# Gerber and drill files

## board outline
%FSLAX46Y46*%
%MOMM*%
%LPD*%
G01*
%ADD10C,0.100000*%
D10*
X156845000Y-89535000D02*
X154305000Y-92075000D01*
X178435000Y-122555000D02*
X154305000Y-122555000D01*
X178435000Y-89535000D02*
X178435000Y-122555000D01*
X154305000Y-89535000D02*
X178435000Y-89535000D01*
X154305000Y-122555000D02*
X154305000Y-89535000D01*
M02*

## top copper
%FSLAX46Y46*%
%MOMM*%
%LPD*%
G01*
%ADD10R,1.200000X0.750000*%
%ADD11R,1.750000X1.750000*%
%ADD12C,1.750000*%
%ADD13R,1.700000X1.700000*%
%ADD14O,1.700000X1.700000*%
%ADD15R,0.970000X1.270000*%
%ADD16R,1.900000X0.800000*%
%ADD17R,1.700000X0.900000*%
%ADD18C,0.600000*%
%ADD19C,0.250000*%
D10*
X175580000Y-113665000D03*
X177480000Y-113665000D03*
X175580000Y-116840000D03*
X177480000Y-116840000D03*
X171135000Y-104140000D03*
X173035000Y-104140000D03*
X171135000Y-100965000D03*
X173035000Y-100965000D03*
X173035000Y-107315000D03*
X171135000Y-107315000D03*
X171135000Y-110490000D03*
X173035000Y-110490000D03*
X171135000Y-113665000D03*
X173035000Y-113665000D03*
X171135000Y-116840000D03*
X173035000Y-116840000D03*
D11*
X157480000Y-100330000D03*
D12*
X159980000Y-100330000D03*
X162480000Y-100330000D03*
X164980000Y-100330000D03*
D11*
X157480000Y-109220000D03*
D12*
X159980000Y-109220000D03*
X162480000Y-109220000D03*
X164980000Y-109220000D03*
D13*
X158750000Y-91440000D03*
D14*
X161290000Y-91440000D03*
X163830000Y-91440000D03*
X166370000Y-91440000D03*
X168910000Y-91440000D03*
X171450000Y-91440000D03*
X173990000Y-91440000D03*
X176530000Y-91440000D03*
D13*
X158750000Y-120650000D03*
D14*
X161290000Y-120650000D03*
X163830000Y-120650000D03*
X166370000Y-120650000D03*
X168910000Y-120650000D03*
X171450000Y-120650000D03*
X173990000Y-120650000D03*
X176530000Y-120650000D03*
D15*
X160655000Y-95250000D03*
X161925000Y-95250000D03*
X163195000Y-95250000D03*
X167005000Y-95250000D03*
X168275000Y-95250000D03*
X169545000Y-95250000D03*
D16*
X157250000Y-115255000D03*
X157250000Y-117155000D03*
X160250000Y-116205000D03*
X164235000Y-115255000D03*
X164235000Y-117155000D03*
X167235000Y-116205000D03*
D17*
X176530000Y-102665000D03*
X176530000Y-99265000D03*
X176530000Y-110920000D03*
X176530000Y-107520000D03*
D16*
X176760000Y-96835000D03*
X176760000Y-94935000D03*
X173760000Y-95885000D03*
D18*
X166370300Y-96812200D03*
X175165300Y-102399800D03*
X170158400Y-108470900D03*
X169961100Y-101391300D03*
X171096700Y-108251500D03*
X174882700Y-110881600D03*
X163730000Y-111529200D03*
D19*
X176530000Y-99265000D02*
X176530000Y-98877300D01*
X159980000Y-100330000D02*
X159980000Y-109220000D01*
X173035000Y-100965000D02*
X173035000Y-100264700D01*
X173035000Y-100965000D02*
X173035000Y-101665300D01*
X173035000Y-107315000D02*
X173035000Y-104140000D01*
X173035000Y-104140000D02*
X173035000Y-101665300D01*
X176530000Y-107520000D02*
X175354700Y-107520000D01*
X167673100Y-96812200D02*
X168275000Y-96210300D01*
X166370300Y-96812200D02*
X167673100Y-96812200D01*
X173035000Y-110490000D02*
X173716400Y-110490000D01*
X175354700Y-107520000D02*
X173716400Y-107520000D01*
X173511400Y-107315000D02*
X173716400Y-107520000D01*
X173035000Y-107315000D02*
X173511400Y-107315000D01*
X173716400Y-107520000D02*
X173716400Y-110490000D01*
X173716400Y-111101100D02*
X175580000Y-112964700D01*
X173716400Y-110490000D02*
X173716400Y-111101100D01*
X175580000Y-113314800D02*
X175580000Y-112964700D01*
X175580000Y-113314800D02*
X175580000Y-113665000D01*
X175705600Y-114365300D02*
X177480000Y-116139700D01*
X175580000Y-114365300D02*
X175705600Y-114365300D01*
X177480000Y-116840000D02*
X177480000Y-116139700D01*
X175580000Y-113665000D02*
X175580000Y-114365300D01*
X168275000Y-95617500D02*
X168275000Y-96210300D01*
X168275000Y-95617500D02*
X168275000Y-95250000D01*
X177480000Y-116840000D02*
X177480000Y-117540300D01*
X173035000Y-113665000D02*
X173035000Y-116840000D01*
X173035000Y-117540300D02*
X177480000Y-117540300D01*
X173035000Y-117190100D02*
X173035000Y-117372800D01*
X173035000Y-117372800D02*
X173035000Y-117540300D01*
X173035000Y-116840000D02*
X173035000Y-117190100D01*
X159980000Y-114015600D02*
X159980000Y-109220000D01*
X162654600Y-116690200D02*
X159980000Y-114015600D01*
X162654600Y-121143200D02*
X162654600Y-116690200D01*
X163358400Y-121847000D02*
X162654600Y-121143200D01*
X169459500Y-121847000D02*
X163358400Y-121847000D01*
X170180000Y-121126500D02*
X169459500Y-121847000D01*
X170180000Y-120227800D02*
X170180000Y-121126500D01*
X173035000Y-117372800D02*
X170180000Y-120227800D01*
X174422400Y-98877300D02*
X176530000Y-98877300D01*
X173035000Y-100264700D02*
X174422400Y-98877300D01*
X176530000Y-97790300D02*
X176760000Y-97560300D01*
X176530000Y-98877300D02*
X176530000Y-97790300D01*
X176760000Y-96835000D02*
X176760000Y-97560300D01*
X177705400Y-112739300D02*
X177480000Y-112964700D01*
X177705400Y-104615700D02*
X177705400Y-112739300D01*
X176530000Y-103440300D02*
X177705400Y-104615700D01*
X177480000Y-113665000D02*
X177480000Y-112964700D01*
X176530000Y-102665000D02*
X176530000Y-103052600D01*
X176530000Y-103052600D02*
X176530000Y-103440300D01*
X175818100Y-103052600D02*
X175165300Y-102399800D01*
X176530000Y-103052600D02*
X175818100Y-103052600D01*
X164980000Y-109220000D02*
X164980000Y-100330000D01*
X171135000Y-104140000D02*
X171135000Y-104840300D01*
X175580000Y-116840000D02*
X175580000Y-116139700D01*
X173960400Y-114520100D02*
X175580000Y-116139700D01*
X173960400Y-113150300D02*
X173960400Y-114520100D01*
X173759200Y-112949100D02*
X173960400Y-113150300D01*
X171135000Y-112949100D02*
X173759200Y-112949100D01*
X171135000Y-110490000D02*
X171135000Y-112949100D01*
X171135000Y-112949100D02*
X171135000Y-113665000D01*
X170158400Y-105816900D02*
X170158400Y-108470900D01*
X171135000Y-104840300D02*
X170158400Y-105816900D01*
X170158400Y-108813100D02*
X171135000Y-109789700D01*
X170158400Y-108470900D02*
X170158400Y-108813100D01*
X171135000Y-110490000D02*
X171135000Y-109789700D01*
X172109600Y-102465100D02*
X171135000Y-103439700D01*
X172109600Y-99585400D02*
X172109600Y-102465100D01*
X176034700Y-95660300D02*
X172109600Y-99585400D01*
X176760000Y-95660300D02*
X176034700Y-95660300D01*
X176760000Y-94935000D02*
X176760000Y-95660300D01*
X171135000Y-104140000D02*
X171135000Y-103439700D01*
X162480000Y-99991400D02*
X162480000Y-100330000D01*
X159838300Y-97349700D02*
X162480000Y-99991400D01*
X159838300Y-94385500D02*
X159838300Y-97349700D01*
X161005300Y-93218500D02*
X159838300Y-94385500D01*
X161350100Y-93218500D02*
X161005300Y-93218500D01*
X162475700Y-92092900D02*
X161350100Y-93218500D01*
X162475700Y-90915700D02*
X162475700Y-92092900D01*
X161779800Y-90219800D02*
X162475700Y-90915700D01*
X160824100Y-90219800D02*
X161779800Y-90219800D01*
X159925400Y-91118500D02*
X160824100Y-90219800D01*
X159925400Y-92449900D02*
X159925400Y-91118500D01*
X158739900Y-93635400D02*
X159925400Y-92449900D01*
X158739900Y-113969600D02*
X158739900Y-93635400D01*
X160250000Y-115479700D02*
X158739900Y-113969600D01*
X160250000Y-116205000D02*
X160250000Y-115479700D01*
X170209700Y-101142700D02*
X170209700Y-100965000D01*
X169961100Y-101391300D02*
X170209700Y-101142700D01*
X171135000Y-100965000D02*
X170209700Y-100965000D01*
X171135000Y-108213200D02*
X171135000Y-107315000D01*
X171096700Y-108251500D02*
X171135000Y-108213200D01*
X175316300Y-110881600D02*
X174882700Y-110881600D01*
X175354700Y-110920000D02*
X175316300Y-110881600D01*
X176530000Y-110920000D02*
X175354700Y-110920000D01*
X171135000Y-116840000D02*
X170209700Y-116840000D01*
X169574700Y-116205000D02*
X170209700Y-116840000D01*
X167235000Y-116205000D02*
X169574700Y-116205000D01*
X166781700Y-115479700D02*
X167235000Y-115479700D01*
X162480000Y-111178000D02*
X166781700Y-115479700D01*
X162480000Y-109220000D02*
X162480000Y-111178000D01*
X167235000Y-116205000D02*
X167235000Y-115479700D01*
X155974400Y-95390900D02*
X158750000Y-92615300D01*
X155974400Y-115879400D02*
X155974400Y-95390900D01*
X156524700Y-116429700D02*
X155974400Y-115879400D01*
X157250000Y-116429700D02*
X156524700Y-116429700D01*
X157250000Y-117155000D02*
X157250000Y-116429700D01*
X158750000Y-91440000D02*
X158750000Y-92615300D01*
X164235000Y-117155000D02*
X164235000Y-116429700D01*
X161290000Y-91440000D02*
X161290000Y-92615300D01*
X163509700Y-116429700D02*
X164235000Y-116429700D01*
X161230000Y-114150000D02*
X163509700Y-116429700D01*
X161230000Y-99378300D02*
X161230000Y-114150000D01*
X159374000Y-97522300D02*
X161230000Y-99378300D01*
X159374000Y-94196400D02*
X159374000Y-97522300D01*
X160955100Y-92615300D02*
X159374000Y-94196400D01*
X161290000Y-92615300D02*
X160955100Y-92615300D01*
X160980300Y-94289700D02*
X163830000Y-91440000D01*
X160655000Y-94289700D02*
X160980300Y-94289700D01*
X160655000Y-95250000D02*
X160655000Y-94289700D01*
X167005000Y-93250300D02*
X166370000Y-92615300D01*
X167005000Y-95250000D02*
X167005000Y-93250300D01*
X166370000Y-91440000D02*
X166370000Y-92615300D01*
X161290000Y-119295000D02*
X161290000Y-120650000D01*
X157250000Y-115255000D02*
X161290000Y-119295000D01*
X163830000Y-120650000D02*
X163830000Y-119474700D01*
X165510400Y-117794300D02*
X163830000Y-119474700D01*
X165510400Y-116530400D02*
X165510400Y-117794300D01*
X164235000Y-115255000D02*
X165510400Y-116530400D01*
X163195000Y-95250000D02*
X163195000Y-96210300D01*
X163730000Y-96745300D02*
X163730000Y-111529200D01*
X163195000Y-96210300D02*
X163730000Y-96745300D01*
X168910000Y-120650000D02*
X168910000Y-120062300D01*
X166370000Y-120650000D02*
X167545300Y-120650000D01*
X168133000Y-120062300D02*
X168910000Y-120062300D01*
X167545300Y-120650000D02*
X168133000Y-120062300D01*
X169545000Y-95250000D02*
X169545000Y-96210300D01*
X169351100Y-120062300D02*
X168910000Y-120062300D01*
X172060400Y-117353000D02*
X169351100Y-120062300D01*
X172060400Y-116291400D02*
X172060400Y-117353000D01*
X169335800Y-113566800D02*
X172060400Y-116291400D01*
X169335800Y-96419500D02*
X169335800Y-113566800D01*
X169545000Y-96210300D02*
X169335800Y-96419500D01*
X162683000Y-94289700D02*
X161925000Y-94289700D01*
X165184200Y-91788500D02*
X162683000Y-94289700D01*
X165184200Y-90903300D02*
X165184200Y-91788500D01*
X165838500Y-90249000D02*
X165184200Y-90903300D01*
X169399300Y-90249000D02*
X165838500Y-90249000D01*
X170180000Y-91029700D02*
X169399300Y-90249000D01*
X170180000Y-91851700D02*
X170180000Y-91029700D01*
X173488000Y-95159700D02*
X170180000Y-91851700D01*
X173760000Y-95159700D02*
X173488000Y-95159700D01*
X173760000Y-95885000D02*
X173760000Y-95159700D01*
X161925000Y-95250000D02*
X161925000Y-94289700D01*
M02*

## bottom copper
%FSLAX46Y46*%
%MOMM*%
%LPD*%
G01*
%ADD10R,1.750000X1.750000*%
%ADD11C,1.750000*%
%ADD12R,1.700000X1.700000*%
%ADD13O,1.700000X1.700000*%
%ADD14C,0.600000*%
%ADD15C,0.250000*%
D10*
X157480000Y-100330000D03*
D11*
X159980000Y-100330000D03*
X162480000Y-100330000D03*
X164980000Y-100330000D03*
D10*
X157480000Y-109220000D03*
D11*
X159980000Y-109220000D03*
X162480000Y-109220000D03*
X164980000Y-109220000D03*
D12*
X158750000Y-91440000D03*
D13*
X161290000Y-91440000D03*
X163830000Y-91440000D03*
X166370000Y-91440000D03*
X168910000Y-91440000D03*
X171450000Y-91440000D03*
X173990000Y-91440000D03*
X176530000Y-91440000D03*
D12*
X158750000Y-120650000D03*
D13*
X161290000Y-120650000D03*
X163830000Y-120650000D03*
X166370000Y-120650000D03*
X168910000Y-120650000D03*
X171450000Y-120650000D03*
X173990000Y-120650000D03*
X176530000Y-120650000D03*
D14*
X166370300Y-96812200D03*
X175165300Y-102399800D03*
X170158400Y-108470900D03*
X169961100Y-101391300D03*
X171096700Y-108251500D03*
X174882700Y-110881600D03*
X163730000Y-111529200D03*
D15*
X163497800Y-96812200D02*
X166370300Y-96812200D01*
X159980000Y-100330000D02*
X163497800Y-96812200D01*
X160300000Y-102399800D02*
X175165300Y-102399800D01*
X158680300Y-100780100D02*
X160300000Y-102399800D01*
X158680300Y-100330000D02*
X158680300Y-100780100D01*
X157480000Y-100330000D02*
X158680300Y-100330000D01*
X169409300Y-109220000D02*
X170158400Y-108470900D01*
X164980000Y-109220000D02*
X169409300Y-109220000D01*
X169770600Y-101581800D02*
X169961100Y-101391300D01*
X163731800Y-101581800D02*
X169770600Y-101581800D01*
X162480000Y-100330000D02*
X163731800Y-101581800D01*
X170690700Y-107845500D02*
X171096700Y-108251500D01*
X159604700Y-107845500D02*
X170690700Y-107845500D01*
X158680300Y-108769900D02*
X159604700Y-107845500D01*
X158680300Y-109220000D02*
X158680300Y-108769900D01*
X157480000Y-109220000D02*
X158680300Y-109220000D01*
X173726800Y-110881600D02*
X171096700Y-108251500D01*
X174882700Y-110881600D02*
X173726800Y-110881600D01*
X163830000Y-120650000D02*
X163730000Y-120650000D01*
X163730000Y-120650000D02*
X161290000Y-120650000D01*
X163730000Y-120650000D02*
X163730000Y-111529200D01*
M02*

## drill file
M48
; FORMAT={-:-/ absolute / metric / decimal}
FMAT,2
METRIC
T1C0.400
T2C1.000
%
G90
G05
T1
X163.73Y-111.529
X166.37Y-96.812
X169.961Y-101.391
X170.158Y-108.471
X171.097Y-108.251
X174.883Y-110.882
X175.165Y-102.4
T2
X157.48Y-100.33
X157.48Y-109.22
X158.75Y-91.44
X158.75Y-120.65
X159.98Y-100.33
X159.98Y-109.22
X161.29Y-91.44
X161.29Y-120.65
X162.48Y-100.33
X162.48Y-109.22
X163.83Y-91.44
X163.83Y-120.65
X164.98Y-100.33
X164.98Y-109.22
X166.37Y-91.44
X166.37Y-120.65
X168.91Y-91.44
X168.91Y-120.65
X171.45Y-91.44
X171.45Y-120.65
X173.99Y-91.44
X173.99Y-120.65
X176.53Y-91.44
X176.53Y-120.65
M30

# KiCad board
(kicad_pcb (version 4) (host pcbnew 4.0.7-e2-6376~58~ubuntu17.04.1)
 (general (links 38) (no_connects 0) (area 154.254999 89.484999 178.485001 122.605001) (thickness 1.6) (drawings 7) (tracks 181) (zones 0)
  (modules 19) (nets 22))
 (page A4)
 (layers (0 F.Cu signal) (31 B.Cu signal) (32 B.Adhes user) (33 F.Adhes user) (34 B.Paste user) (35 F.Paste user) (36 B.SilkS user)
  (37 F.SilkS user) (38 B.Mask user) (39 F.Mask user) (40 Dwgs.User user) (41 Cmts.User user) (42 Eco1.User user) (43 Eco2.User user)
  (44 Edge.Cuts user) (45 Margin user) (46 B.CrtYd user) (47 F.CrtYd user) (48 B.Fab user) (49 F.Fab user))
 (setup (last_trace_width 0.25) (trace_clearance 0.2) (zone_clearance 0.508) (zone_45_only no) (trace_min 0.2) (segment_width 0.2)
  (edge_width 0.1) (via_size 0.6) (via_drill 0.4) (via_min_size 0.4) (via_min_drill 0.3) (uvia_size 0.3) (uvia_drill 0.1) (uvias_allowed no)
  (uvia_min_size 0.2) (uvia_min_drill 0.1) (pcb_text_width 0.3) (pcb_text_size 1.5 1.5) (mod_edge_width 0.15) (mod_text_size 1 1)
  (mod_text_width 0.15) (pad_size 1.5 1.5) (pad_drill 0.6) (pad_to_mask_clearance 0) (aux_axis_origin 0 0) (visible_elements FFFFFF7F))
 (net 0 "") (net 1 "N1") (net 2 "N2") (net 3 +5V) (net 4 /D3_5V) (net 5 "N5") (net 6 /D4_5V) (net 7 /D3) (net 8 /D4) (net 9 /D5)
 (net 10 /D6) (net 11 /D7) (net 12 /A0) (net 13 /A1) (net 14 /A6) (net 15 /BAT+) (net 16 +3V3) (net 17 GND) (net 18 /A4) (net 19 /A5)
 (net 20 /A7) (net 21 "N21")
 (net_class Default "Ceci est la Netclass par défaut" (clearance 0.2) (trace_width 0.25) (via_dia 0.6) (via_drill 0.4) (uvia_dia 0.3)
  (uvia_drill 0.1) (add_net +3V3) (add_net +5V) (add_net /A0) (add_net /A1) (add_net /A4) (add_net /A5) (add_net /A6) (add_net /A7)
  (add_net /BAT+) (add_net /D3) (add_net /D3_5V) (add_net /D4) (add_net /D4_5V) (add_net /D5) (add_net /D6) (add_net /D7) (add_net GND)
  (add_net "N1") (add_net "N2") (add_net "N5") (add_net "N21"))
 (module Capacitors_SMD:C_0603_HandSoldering (layer F.Cu) (at 176.53 113.665)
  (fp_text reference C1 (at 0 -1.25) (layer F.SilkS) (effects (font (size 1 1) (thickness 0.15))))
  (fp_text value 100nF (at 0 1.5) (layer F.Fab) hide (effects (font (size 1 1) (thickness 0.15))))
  (pad 1 smd rect (at -0.95 0) (size 1.2 0.75) (layers F.Cu F.Paste F.Mask) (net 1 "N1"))
  (pad 2 smd rect (at 0.95 0) (size 1.2 0.75) (layers F.Cu F.Paste F.Mask) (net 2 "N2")))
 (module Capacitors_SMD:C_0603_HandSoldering (layer F.Cu) (at 176.53 116.84)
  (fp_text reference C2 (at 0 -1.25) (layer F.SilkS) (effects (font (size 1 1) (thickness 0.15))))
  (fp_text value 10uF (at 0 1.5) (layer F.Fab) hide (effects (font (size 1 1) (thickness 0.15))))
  (pad 1 smd rect (at -0.95 0) (size 1.2 0.75) (layers F.Cu F.Paste F.Mask) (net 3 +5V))
  (pad 2 smd rect (at 0.95 0) (size 1.2 0.75) (layers F.Cu F.Paste F.Mask) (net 1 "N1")))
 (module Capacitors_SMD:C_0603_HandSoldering (layer F.Cu) (at 172.085 104.14)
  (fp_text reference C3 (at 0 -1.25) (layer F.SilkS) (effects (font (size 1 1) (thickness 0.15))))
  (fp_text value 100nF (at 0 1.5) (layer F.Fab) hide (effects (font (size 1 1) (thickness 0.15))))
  (pad 1 smd rect (at -0.95 0) (size 1.2 0.75) (layers F.Cu F.Paste F.Mask) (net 3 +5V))
  (pad 2 smd rect (at 0.95 0) (size 1.2 0.75) (layers F.Cu F.Paste F.Mask) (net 1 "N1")))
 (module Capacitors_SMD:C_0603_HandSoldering (layer F.Cu) (at 172.085 100.965)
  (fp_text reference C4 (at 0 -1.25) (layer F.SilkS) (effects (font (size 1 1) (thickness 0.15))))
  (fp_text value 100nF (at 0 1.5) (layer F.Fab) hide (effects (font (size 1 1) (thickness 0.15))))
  (pad 1 smd rect (at -0.95 0) (size 1.2 0.75) (layers F.Cu F.Paste F.Mask) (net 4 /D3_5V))
  (pad 2 smd rect (at 0.95 0) (size 1.2 0.75) (layers F.Cu F.Paste F.Mask) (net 1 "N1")))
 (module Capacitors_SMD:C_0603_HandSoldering (layer F.Cu) (at 172.085 107.315 180)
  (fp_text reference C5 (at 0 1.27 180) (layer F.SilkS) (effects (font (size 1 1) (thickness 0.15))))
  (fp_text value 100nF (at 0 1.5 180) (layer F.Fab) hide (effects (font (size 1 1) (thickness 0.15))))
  (pad 1 smd rect (at -0.95 0 180) (size 1.2 0.75) (layers F.Cu F.Paste F.Mask) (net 1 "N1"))
  (pad 2 smd rect (at 0.95 0 180) (size 1.2 0.75) (layers F.Cu F.Paste F.Mask) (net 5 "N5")))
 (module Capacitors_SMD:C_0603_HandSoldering (layer F.Cu) (at 172.085 110.49)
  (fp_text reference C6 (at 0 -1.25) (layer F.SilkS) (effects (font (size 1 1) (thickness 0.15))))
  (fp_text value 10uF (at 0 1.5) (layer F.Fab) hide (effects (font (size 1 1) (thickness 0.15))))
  (pad 1 smd rect (at -0.95 0) (size 1.2 0.75) (layers F.Cu F.Paste F.Mask) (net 3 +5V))
  (pad 2 smd rect (at 0.95 0) (size 1.2 0.75) (layers F.Cu F.Paste F.Mask) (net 1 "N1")))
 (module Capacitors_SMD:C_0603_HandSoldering (layer F.Cu) (at 172.085 113.665)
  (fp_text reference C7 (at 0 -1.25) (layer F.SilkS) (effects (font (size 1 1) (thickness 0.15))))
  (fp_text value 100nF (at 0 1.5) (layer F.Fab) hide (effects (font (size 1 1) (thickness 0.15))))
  (pad 1 smd rect (at -0.95 0) (size 1.2 0.75) (layers F.Cu F.Paste F.Mask) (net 3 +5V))
  (pad 2 smd rect (at 0.95 0) (size 1.2 0.75) (layers F.Cu F.Paste F.Mask) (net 1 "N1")))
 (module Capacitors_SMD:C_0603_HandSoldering (layer F.Cu) (at 172.085 116.84)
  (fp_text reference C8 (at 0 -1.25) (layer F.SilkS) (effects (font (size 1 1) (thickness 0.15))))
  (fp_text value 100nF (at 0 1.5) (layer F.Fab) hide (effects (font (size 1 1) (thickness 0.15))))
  (pad 1 smd rect (at -0.95 0) (size 1.2 0.75) (layers F.Cu F.Paste F.Mask) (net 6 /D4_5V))
  (pad 2 smd rect (at 0.95 0) (size 1.2 0.75) (layers F.Cu F.Paste F.Mask) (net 1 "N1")))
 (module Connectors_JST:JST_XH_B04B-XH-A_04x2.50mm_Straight (layer F.Cu) (at 157.48 100.33)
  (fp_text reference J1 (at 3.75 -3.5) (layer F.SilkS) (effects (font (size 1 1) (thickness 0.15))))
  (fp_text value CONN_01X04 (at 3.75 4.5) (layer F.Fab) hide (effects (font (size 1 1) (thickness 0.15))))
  (pad 1 thru_hole rect (at 0 0) (size 1.75 1.75) (drill 1) (layers *.Cu *.Mask) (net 2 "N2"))
  (pad 2 thru_hole circle (at 2.5 0) (size 1.75 1.75) (drill 1) (layers *.Cu *.Mask) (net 1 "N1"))
  (pad 3 thru_hole circle (at 5 0) (size 1.75 1.75) (drill 1) (layers *.Cu *.Mask) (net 4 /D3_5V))
  (pad 4 thru_hole circle (at 7.5 0) (size 1.75 1.75) (drill 1) (layers *.Cu *.Mask) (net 3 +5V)))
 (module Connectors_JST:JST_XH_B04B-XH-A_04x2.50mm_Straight (layer F.Cu) (at 157.48 109.22)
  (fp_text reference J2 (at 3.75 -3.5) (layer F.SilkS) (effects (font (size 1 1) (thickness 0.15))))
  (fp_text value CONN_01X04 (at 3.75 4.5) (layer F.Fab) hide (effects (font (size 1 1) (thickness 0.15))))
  (pad 1 thru_hole rect (at 0 0) (size 1.75 1.75) (drill 1) (layers *.Cu *.Mask) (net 5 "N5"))
  (pad 2 thru_hole circle (at 2.5 0) (size 1.75 1.75) (drill 1) (layers *.Cu *.Mask) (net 1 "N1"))
  (pad 3 thru_hole circle (at 5 0) (size 1.75 1.75) (drill 1) (layers *.Cu *.Mask) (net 6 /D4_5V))
  (pad 4 thru_hole circle (at 7.5 0) (size 1.75 1.75) (drill 1) (layers *.Cu *.Mask) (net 3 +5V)))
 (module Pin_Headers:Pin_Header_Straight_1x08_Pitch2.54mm (layer B.Cu) (at 158.75 91.44 270)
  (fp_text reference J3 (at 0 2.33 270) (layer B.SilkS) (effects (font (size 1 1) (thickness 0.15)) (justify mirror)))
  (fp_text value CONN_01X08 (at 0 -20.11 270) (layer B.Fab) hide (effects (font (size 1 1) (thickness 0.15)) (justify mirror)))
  (pad 1 thru_hole rect (at 0 0 270) (size 1.7 1.7) (drill 1) (layers *.Cu *.Mask) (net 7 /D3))
  (pad 2 thru_hole oval (at 0 -2.54 270) (size 1.7 1.7) (drill 1) (layers *.Cu *.Mask) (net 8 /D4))
  (pad 3 thru_hole oval (at 0 -5.08 270) (size 1.7 1.7) (drill 1) (layers *.Cu *.Mask) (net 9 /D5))
  (pad 4 thru_hole oval (at 0 -7.62 270) (size 1.7 1.7) (drill 1) (layers *.Cu *.Mask) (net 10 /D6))
  (pad 5 thru_hole oval (at 0 -10.16 270) (size 1.7 1.7) (drill 1) (layers *.Cu *.Mask) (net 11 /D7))
  (pad 6 thru_hole oval (at 0 -12.7 270) (size 1.7 1.7) (drill 1) (layers *.Cu *.Mask) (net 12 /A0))
  (pad 7 thru_hole oval (at 0 -15.24 270) (size 1.7 1.7) (drill 1) (layers *.Cu *.Mask) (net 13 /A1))
  (pad 8 thru_hole oval (at 0 -17.78 270) (size 1.7 1.7) (drill 1) (layers *.Cu *.Mask) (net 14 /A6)))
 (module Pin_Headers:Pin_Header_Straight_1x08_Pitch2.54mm (layer B.Cu) (at 158.75 120.65 270)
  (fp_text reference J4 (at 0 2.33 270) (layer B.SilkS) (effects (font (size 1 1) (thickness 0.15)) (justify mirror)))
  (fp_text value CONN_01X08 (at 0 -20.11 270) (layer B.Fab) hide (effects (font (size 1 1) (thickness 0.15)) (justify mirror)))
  (pad 1 thru_hole rect (at 0 0 270) (size 1.7 1.7) (drill 1) (layers *.Cu *.Mask) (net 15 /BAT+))
  (pad 2 thru_hole oval (at 0 -2.54 270) (size 1.7 1.7) (drill 1) (layers *.Cu *.Mask) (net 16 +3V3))
  (pad 3 thru_hole oval (at 0 -5.08 270) (size 1.7 1.7) (drill 1) (layers *.Cu *.Mask) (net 16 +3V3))
  (pad 4 thru_hole oval (at 0 -7.62 270) (size 1.7 1.7) (drill 1) (layers *.Cu *.Mask) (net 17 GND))
  (pad 5 thru_hole oval (at 0 -10.16 270) (size 1.7 1.7) (drill 1) (layers *.Cu *.Mask) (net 17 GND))
  (pad 6 thru_hole oval (at 0 -12.7 270) (size 1.7 1.7) (drill 1) (layers *.Cu *.Mask) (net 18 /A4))
  (pad 7 thru_hole oval (at 0 -15.24 270) (size 1.7 1.7) (drill 1) (layers *.Cu *.Mask) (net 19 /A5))
  (pad 8 thru_hole oval (at 0 -17.78 270) (size 1.7 1.7) (drill 1) (layers *.Cu *.Mask) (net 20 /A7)))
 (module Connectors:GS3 (layer F.Cu) (at 161.925 95.25 90)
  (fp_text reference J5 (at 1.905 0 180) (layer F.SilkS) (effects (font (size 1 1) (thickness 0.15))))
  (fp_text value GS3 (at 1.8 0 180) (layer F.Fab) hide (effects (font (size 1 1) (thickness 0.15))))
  (pad 1 smd rect (at 0 -1.27 90) (size 1.27 0.97) (layers F.Cu F.Paste F.Mask) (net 9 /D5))
  (pad 2 smd rect (at 0 0 90) (size 1.27 0.97) (layers F.Cu F.Paste F.Mask) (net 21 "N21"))
  (pad 3 smd rect (at 0 1.27 90) (size 1.27 0.97) (layers F.Cu F.Paste F.Mask) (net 16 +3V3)))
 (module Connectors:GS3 (layer F.Cu) (at 168.275 95.25 90)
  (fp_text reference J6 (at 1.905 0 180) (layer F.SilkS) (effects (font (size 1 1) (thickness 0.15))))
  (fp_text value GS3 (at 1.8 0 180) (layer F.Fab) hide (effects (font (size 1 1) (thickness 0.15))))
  (pad 1 smd rect (at 0 -1.27 90) (size 1.27 0.97) (layers F.Cu F.Paste F.Mask) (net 10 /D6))
  (pad 2 smd rect (at 0 0 90) (size 1.27 0.97) (layers F.Cu F.Paste F.Mask) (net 1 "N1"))
  (pad 3 smd rect (at 0 1.27 90) (size 1.27 0.97) (layers F.Cu F.Paste F.Mask) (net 17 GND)))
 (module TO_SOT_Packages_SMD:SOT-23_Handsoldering (layer F.Cu) (at 158.75 116.205)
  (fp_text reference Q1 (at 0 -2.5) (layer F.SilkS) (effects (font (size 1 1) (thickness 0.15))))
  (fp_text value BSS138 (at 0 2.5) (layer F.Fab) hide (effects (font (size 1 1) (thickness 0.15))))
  (pad 1 smd rect (at -1.5 -0.95) (size 1.9 0.8) (layers F.Cu F.Paste F.Mask) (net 16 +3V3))
  (pad 2 smd rect (at -1.5 0.95) (size 1.9 0.8) (layers F.Cu F.Paste F.Mask) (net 7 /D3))
  (pad 3 smd rect (at 1.5 0) (size 1.9 0.8) (layers F.Cu F.Paste F.Mask) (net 4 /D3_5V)))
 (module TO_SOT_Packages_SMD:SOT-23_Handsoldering (layer F.Cu) (at 165.735 116.205)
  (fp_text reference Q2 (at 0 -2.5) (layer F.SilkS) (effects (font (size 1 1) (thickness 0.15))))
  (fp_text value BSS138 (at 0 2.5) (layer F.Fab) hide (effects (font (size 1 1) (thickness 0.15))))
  (pad 1 smd rect (at -1.5 -0.95) (size 1.9 0.8) (layers F.Cu F.Paste F.Mask) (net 16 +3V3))
  (pad 2 smd rect (at -1.5 0.95) (size 1.9 0.8) (layers F.Cu F.Paste F.Mask) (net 8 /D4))
  (pad 3 smd rect (at 1.5 0) (size 1.9 0.8) (layers F.Cu F.Paste F.Mask) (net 6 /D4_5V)))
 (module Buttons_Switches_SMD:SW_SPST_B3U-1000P (layer F.Cu) (at 176.53 100.965 90)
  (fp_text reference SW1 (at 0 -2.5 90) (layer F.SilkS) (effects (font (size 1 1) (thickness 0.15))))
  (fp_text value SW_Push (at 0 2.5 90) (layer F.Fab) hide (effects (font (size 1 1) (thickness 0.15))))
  (pad 1 smd rect (at -1.7 0 90) (size 0.9 1.7) (layers F.Cu F.Paste F.Mask) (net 2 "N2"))
  (pad 2 smd rect (at 1.7 0 90) (size 0.9 1.7) (layers F.Cu F.Paste F.Mask) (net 1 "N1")))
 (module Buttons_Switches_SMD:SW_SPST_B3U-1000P (layer F.Cu) (at 176.53 109.22 90)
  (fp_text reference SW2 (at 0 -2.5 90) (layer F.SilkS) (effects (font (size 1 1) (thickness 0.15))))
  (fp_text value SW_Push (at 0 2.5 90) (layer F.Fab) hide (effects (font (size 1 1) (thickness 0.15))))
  (pad 1 smd rect (at -1.7 0 90) (size 0.9 1.7) (layers F.Cu F.Paste F.Mask) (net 5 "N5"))
  (pad 2 smd rect (at 1.7 0 90) (size 0.9 1.7) (layers F.Cu F.Paste F.Mask) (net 1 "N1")))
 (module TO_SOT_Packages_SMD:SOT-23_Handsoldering (layer F.Cu) (at 175.26 95.885 180)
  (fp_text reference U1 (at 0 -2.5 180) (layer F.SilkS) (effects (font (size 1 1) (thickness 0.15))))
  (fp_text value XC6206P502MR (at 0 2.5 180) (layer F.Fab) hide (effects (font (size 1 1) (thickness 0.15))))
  (pad 1 smd rect (at -1.5 -0.95 180) (size 1.9 0.8) (layers F.Cu F.Paste F.Mask) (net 1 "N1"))
  (pad 2 smd rect (at -1.5 0.95 180) (size 1.9 0.8) (layers F.Cu F.Paste F.Mask) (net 3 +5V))
  (pad 3 smd rect (at 1.5 0 180) (size 1.9 0.8) (layers F.Cu F.Paste F.Mask) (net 21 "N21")))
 (gr_line (start 156.845 89.535) (end 154.305 92.075) (angle 90) (layer Edge.Cuts) (width 0.1))
 (gr_line (start 178.435 122.555) (end 154.305 122.555) (angle 90) (layer Edge.Cuts) (width 0.1))
 (gr_line (start 178.435 89.535) (end 178.435 122.555) (angle 90) (layer Edge.Cuts) (width 0.1))
 (gr_line (start 154.305 89.535) (end 178.435 89.535) (angle 90) (layer Edge.Cuts) (width 0.1))
 (gr_line (start 154.305 122.555) (end 154.305 89.535) (angle 90) (layer Edge.Cuts) (width 0.1))
 (via (at 166.3703 96.8122) (size 0.6) (layers F.Cu B.Cu) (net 1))
 (segment (start 176.53 99.265) (end 176.53 98.8773) (width 0.25) (layer F.Cu) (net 1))
 (segment (start 159.98 100.33) (end 159.98 109.22) (width 0.25) (layer F.Cu) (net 1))
 (segment (start 173.035 100.965) (end 173.035 100.2647) (width 0.25) (layer F.Cu) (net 1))
 (segment (start 173.035 100.965) (end 173.035 101.6653) (width 0.25) (layer F.Cu) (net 1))
 (segment (start 173.035 107.315) (end 173.035 104.14) (width 0.25) (layer F.Cu) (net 1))
 (segment (start 173.035 104.14) (end 173.035 101.6653) (width 0.25) (layer F.Cu) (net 1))
 (segment (start 176.53 107.52) (end 175.3547 107.52) (width 0.25) (layer F.Cu) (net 1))
 (segment (start 163.4978 96.8122) (end 166.3703 96.8122) (width 0.25) (layer B.Cu) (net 1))
 (segment (start 159.98 100.33) (end 163.4978 96.8122) (width 0.25) (layer B.Cu) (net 1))
 (segment (start 167.6731 96.8122) (end 168.275 96.2103) (width 0.25) (layer F.Cu) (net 1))
 (segment (start 166.3703 96.8122) (end 167.6731 96.8122) (width 0.25) (layer F.Cu) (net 1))
 (segment (start 173.035 110.49) (end 173.7164 110.49) (width 0.25) (layer F.Cu) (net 1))
 (segment (start 175.3547 107.52) (end 173.7164 107.52) (width 0.25) (layer F.Cu) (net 1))
 (segment (start 173.5114 107.315) (end 173.7164 107.52) (width 0.25) (layer F.Cu) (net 1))
 (segment (start 173.035 107.315) (end 173.5114 107.315) (width 0.25) (layer F.Cu) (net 1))
 (segment (start 173.7164 107.52) (end 173.7164 110.49) (width 0.25) (layer F.Cu) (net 1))
 (segment (start 173.7164 111.1011) (end 175.58 112.9647) (width 0.25) (layer F.Cu) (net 1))
 (segment (start 173.7164 110.49) (end 173.7164 111.1011) (width 0.25) (layer F.Cu) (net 1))
 (segment (start 175.58 113.3148) (end 175.58 112.9647) (width 0.25) (layer F.Cu) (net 1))
 (segment (start 175.58 113.3148) (end 175.58 113.665) (width 0.25) (layer F.Cu) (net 1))
 (segment (start 175.7056 114.3653) (end 177.48 116.1397) (width 0.25) (layer F.Cu) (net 1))
 (segment (start 175.58 114.3653) (end 175.7056 114.3653) (width 0.25) (layer F.Cu) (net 1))
 (segment (start 177.48 116.84) (end 177.48 116.1397) (width 0.25) (layer F.Cu) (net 1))
 (segment (start 175.58 113.665) (end 175.58 114.3653) (width 0.25) (layer F.Cu) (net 1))
 (segment (start 168.275 95.6175) (end 168.275 96.2103) (width 0.25) (layer F.Cu) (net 1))
 (segment (start 168.275 95.6175) (end 168.275 95.25) (width 0.25) (layer F.Cu) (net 1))
 (segment (start 177.48 116.84) (end 177.48 117.5403) (width 0.25) (layer F.Cu) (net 1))
 (segment (start 173.035 113.665) (end 173.035 116.84) (width 0.25) (layer F.Cu) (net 1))
 (segment (start 173.035 117.5403) (end 177.48 117.5403) (width 0.25) (layer F.Cu) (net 1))
 (segment (start 173.035 117.1901) (end 173.035 117.3728) (width 0.25) (layer F.Cu) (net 1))
 (segment (start 173.035 117.3728) (end 173.035 117.5403) (width 0.25) (layer F.Cu) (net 1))
 (segment (start 173.035 116.84) (end 173.035 117.1901) (width 0.25) (layer F.Cu) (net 1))
 (segment (start 159.98 114.0156) (end 159.98 109.22) (width 0.25) (layer F.Cu) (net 1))
 (segment (start 162.6546 116.6902) (end 159.98 114.0156) (width 0.25) (layer F.Cu) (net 1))
 (segment (start 162.6546 121.1432) (end 162.6546 116.6902) (width 0.25) (layer F.Cu) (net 1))
 (segment (start 163.3584 121.847) (end 162.6546 121.1432) (width 0.25) (layer F.Cu) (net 1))
 (segment (start 169.4595 121.847) (end 163.3584 121.847) (width 0.25) (layer F.Cu) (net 1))
 (segment (start 170.18 121.1265) (end 169.4595 121.847) (width 0.25) (layer F.Cu) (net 1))
 (segment (start 170.18 120.2278) (end 170.18 121.1265) (width 0.25) (layer F.Cu) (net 1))
 (segment (start 173.035 117.3728) (end 170.18 120.2278) (width 0.25) (layer F.Cu) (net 1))
 (segment (start 174.4224 98.8773) (end 176.53 98.8773) (width 0.25) (layer F.Cu) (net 1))
 (segment (start 173.035 100.2647) (end 174.4224 98.8773) (width 0.25) (layer F.Cu) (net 1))
 (segment (start 176.53 97.7903) (end 176.76 97.5603) (width 0.25) (layer F.Cu) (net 1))
 (segment (start 176.53 98.8773) (end 176.53 97.7903) (width 0.25) (layer F.Cu) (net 1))
 (segment (start 176.76 96.835) (end 176.76 97.5603) (width 0.25) (layer F.Cu) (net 1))
 (via (at 175.1653 102.3998) (size 0.6) (layers F.Cu B.Cu) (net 2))
 (segment (start 177.7054 112.7393) (end 177.48 112.9647) (width 0.25) (layer F.Cu) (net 2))
 (segment (start 177.7054 104.6157) (end 177.7054 112.7393) (width 0.25) (layer F.Cu) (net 2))
 (segment (start 176.53 103.4403) (end 177.7054 104.6157) (width 0.25) (layer F.Cu) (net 2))
 (segment (start 177.48 113.665) (end 177.48 112.9647) (width 0.25) (layer F.Cu) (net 2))
 (segment (start 176.53 102.665) (end 176.53 103.0526) (width 0.25) (layer F.Cu) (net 2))
 (segment (start 176.53 103.0526) (end 176.53 103.4403) (width 0.25) (layer F.Cu) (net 2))
 (segment (start 160.3 102.3998) (end 175.1653 102.3998) (width 0.25) (layer B.Cu) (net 2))
 (segment (start 158.6803 100.7801) (end 160.3 102.3998) (width 0.25) (layer B.Cu) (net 2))
 (segment (start 158.6803 100.33) (end 158.6803 100.7801) (width 0.25) (layer B.Cu) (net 2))
 (segment (start 175.8181 103.0526) (end 175.1653 102.3998) (width 0.25) (layer F.Cu) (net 2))
 (segment (start 176.53 103.0526) (end 175.8181 103.0526) (width 0.25) (layer F.Cu) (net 2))
 (segment (start 157.48 100.33) (end 158.6803 100.33) (width 0.25) (layer B.Cu) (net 2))
 (via (at 170.1584 108.4709) (size 0.6) (layers F.Cu B.Cu) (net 3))
 (segment (start 164.98 109.22) (end 164.98 100.33) (width 0.25) (layer F.Cu) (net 3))
 (segment (start 171.135 104.14) (end 171.135 104.8403) (width 0.25) (layer F.Cu) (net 3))
 (segment (start 169.4093 109.22) (end 170.1584 108.4709) (width 0.25) (layer B.Cu) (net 3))
 (segment (start 164.98 109.22) (end 169.4093 109.22) (width 0.25) (layer B.Cu) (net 3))
 (segment (start 175.58 116.84) (end 175.58 116.1397) (width 0.25) (layer F.Cu) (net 3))
 (segment (start 173.9604 114.5201) (end 175.58 116.1397) (width 0.25) (layer F.Cu) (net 3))
 (segment (start 173.9604 113.1503) (end 173.9604 114.5201) (width 0.25) (layer F.Cu) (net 3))
 (segment (start 173.7592 112.9491) (end 173.9604 113.1503) (width 0.25) (layer F.Cu) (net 3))
 (segment (start 171.135 112.9491) (end 173.7592 112.9491) (width 0.25) (layer F.Cu) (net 3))
 (segment (start 171.135 110.49) (end 171.135 112.9491) (width 0.25) (layer F.Cu) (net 3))
 (segment (start 171.135 112.9491) (end 171.135 113.665) (width 0.25) (layer F.Cu) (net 3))
 (segment (start 170.1584 105.8169) (end 170.1584 108.4709) (width 0.25) (layer F.Cu) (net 3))
 (segment (start 171.135 104.8403) (end 170.1584 105.8169) (width 0.25) (layer F.Cu) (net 3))
 (segment (start 170.1584 108.8131) (end 171.135 109.7897) (width 0.25) (layer F.Cu) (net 3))
 (segment (start 170.1584 108.4709) (end 170.1584 108.8131) (width 0.25) (layer F.Cu) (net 3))
 (segment (start 171.135 110.49) (end 171.135 109.7897) (width 0.25) (layer F.Cu) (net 3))
 (segment (start 172.1096 102.4651) (end 171.135 103.4397) (width 0.25) (layer F.Cu) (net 3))
 (segment (start 172.1096 99.5854) (end 172.1096 102.4651) (width 0.25) (layer F.Cu) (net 3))
 (segment (start 176.0347 95.6603) (end 172.1096 99.5854) (width 0.25) (layer F.Cu) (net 3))
 (segment (start 176.76 95.6603) (end 176.0347 95.6603) (width 0.25) (layer F.Cu) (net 3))
 (segment (start 176.76 94.935) (end 176.76 95.6603) (width 0.25) (layer F.Cu) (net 3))
 (segment (start 171.135 104.14) (end 171.135 103.4397) (width 0.25) (layer F.Cu) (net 3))
 (via (at 169.9611 101.3913) (size 0.6) (layers F.Cu B.Cu) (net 4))
 (segment (start 162.48 99.9914) (end 162.48 100.33) (width 0.25) (layer F.Cu) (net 4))
 (segment (start 159.8383 97.3497) (end 162.48 99.9914) (width 0.25) (layer F.Cu) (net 4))
 (segment (start 159.8383 94.3855) (end 159.8383 97.3497) (width 0.25) (layer F.Cu) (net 4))
 (segment (start 161.0053 93.2185) (end 159.8383 94.3855) (width 0.25) (layer F.Cu) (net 4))
 (segment (start 161.3501 93.2185) (end 161.0053 93.2185) (width 0.25) (layer F.Cu) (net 4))
 (segment (start 162.4757 92.0929) (end 161.3501 93.2185) (width 0.25) (layer F.Cu) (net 4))
 (segment (start 162.4757 90.9157) (end 162.4757 92.0929) (width 0.25) (layer F.Cu) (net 4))
 (segment (start 161.7798 90.2198) (end 162.4757 90.9157) (width 0.25) (layer F.Cu) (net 4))
 (segment (start 160.8241 90.2198) (end 161.7798 90.2198) (width 0.25) (layer F.Cu) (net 4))
 (segment (start 159.9254 91.1185) (end 160.8241 90.2198) (width 0.25) (layer F.Cu) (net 4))
 (segment (start 159.9254 92.4499) (end 159.9254 91.1185) (width 0.25) (layer F.Cu) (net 4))
 (segment (start 158.7399 93.6354) (end 159.9254 92.4499) (width 0.25) (layer F.Cu) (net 4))
 (segment (start 158.7399 113.9696) (end 158.7399 93.6354) (width 0.25) (layer F.Cu) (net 4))
 (segment (start 160.25 115.4797) (end 158.7399 113.9696) (width 0.25) (layer F.Cu) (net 4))
 (segment (start 160.25 116.205) (end 160.25 115.4797) (width 0.25) (layer F.Cu) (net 4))
 (segment (start 169.7706 101.5818) (end 169.9611 101.3913) (width 0.25) (layer B.Cu) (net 4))
 (segment (start 163.7318 101.5818) (end 169.7706 101.5818) (width 0.25) (layer B.Cu) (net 4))
 (segment (start 162.48 100.33) (end 163.7318 101.5818) (width 0.25) (layer B.Cu) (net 4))
 (segment (start 170.2097 101.1427) (end 170.2097 100.965) (width 0.25) (layer F.Cu) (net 4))
 (segment (start 169.9611 101.3913) (end 170.2097 101.1427) (width 0.25) (layer F.Cu) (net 4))
 (segment (start 171.135 100.965) (end 170.2097 100.965) (width 0.25) (layer F.Cu) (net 4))
 (via (at 171.0967 108.2515) (size 0.6) (layers F.Cu B.Cu) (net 5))
 (via (at 174.8827 110.8816) (size 0.6) (layers F.Cu B.Cu) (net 5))
 (segment (start 170.6907 107.8455) (end 171.0967 108.2515) (width 0.25) (layer B.Cu) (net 5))
 (segment (start 159.6047 107.8455) (end 170.6907 107.8455) (width 0.25) (layer B.Cu) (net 5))
 (segment (start 158.6803 108.7699) (end 159.6047 107.8455) (width 0.25) (layer B.Cu) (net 5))
 (segment (start 158.6803 109.22) (end 158.6803 108.7699) (width 0.25) (layer B.Cu) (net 5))
 (segment (start 171.135 108.2132) (end 171.135 107.315) (width 0.25) (layer F.Cu) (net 5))
 (segment (start 171.0967 108.2515) (end 171.135 108.2132) (width 0.25) (layer F.Cu) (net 5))
 (segment (start 157.48 109.22) (end 158.6803 109.22) (width 0.25) (layer B.Cu) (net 5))
 (segment (start 175.3163 110.8816) (end 174.8827 110.8816) (width 0.25) (layer F.Cu) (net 5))
 (segment (start 175.3547 110.92) (end 175.3163 110.8816) (width 0.25) (layer F.Cu) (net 5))
 (segment (start 173.7268 110.8816) (end 171.0967 108.2515) (width 0.25) (layer B.Cu) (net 5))
 (segment (start 174.8827 110.8816) (end 173.7268 110.8816) (width 0.25) (layer B.Cu) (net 5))
 (segment (start 176.53 110.92) (end 175.3547 110.92) (width 0.25) (layer F.Cu) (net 5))
 (segment (start 171.135 116.84) (end 170.2097 116.84) (width 0.25) (layer F.Cu) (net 6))
 (segment (start 169.5747 116.205) (end 170.2097 116.84) (width 0.25) (layer F.Cu) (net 6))
 (segment (start 167.235 116.205) (end 169.5747 116.205) (width 0.25) (layer F.Cu) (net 6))
 (segment (start 166.7817 115.4797) (end 167.235 115.4797) (width 0.25) (layer F.Cu) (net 6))
 (segment (start 162.48 111.178) (end 166.7817 115.4797) (width 0.25) (layer F.Cu) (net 6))
 (segment (start 162.48 109.22) (end 162.48 111.178) (width 0.25) (layer F.Cu) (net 6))
 (segment (start 167.235 116.205) (end 167.235 115.4797) (width 0.25) (layer F.Cu) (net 6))
 (segment (start 155.9744 95.3909) (end 158.75 92.6153) (width 0.25) (layer F.Cu) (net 7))
 (segment (start 155.9744 115.8794) (end 155.9744 95.3909) (width 0.25) (layer F.Cu) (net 7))
 (segment (start 156.5247 116.4297) (end 155.9744 115.8794) (width 0.25) (layer F.Cu) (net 7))
 (segment (start 157.25 116.4297) (end 156.5247 116.4297) (width 0.25) (layer F.Cu) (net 7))
 (segment (start 157.25 117.155) (end 157.25 116.4297) (width 0.25) (layer F.Cu) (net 7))
 (segment (start 158.75 91.44) (end 158.75 92.6153) (width 0.25) (layer F.Cu) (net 7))
 (segment (start 164.235 117.155) (end 164.235 116.4297) (width 0.25) (layer F.Cu) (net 8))
 (segment (start 161.29 91.44) (end 161.29 92.6153) (width 0.25) (layer F.Cu) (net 8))
 (segment (start 163.5097 116.4297) (end 164.235 116.4297) (width 0.25) (layer F.Cu) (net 8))
 (segment (start 161.23 114.15) (end 163.5097 116.4297) (width 0.25) (layer F.Cu) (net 8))
 (segment (start 161.23 99.3783) (end 161.23 114.15) (width 0.25) (layer F.Cu) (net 8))
 (segment (start 159.374 97.5223) (end 161.23 99.3783) (width 0.25) (layer F.Cu) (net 8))
 (segment (start 159.374 94.1964) (end 159.374 97.5223) (width 0.25) (layer F.Cu) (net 8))
 (segment (start 160.9551 92.6153) (end 159.374 94.1964) (width 0.25) (layer F.Cu) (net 8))
 (segment (start 161.29 92.6153) (end 160.9551 92.6153) (width 0.25) (layer F.Cu) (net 8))
 (segment (start 160.9803 94.2897) (end 163.83 91.44) (width 0.25) (layer F.Cu) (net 9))
 (segment (start 160.655 94.2897) (end 160.9803 94.2897) (width 0.25) (layer F.Cu) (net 9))
 (segment (start 160.655 95.25) (end 160.655 94.2897) (width 0.25) (layer F.Cu) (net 9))
 (segment (start 167.005 93.2503) (end 166.37 92.6153) (width 0.25) (layer F.Cu) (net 10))
 (segment (start 167.005 95.25) (end 167.005 93.2503) (width 0.25) (layer F.Cu) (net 10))
 (segment (start 166.37 91.44) (end 166.37 92.6153) (width 0.25) (layer F.Cu) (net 10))
 (via (at 163.73 111.5292) (size 0.6) (layers F.Cu B.Cu) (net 16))
 (segment (start 161.29 119.295) (end 161.29 120.65) (width 0.25) (layer F.Cu) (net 16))
 (segment (start 157.25 115.255) (end 161.29 119.295) (width 0.25) (layer F.Cu) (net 16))
 (segment (start 163.83 120.65) (end 163.83 119.4747) (width 0.25) (layer F.Cu) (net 16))
 (segment (start 165.5104 117.7943) (end 163.83 119.4747) (width 0.25) (layer F.Cu) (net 16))
 (segment (start 165.5104 116.5304) (end 165.5104 117.7943) (width 0.25) (layer F.Cu) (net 16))
 (segment (start 164.235 115.255) (end 165.5104 116.5304) (width 0.25) (layer F.Cu) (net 16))
 (segment (start 163.195 95.25) (end 163.195 96.2103) (width 0.25) (layer F.Cu) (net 16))
 (segment (start 163.83 120.65) (end 163.73 120.65) (width 0.25) (layer B.Cu) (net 16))
 (segment (start 163.73 120.65) (end 161.29 120.65) (width 0.25) (layer B.Cu) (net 16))
 (segment (start 163.73 120.65) (end 163.73 111.5292) (width 0.25) (layer B.Cu) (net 16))
 (segment (start 163.73 96.7453) (end 163.73 111.5292) (width 0.25) (layer F.Cu) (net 16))
 (segment (start 163.195 96.2103) (end 163.73 96.7453) (width 0.25) (layer F.Cu) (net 16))
 (segment (start 168.91 120.65) (end 168.91 120.0623) (width 0.25) (layer F.Cu) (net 17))
 (segment (start 166.37 120.65) (end 167.5453 120.65) (width 0.25) (layer F.Cu) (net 17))
 (segment (start 168.133 120.0623) (end 168.91 120.0623) (width 0.25) (layer F.Cu) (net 17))
 (segment (start 167.5453 120.65) (end 168.133 120.0623) (width 0.25) (layer F.Cu) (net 17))
 (segment (start 169.545 95.25) (end 169.545 96.2103) (width 0.25) (layer F.Cu) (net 17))
 (segment (start 169.3511 120.0623) (end 168.91 120.0623) (width 0.25) (layer F.Cu) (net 17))
 (segment (start 172.0604 117.353) (end 169.3511 120.0623) (width 0.25) (layer F.Cu) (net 17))
 (segment (start 172.0604 116.2914) (end 172.0604 117.353) (width 0.25) (layer F.Cu) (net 17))
 (segment (start 169.3358 113.5668) (end 172.0604 116.2914) (width 0.25) (layer F.Cu) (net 17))
 (segment (start 169.3358 96.4195) (end 169.3358 113.5668) (width 0.25) (layer F.Cu) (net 17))
 (segment (start 169.545 96.2103) (end 169.3358 96.4195) (width 0.25) (layer F.Cu) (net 17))
 (segment (start 162.683 94.2897) (end 161.925 94.2897) (width 0.25) (layer F.Cu) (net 21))
 (segment (start 165.1842 91.7885) (end 162.683 94.2897) (width 0.25) (layer F.Cu) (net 21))
 (segment (start 165.1842 90.9033) (end 165.1842 91.7885) (width 0.25) (layer F.Cu) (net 21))
 (segment (start 165.8385 90.249) (end 165.1842 90.9033) (width 0.25) (layer F.Cu) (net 21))
 (segment (start 169.3993 90.249) (end 165.8385 90.249) (width 0.25) (layer F.Cu) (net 21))
 (segment (start 170.18 91.0297) (end 169.3993 90.249) (width 0.25) (layer F.Cu) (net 21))
 (segment (start 170.18 91.8517) (end 170.18 91.0297) (width 0.25) (layer F.Cu) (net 21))
 (segment (start 173.488 95.1597) (end 170.18 91.8517) (width 0.25) (layer F.Cu) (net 21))
 (segment (start 173.76 95.1597) (end 173.488 95.1597) (width 0.25) (layer F.Cu) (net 21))
 (segment (start 173.76 95.885) (end 173.76 95.1597) (width 0.25) (layer F.Cu) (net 21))
 (segment (start 161.925 95.25) (end 161.925 94.2897) (width 0.25) (layer F.Cu) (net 21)))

